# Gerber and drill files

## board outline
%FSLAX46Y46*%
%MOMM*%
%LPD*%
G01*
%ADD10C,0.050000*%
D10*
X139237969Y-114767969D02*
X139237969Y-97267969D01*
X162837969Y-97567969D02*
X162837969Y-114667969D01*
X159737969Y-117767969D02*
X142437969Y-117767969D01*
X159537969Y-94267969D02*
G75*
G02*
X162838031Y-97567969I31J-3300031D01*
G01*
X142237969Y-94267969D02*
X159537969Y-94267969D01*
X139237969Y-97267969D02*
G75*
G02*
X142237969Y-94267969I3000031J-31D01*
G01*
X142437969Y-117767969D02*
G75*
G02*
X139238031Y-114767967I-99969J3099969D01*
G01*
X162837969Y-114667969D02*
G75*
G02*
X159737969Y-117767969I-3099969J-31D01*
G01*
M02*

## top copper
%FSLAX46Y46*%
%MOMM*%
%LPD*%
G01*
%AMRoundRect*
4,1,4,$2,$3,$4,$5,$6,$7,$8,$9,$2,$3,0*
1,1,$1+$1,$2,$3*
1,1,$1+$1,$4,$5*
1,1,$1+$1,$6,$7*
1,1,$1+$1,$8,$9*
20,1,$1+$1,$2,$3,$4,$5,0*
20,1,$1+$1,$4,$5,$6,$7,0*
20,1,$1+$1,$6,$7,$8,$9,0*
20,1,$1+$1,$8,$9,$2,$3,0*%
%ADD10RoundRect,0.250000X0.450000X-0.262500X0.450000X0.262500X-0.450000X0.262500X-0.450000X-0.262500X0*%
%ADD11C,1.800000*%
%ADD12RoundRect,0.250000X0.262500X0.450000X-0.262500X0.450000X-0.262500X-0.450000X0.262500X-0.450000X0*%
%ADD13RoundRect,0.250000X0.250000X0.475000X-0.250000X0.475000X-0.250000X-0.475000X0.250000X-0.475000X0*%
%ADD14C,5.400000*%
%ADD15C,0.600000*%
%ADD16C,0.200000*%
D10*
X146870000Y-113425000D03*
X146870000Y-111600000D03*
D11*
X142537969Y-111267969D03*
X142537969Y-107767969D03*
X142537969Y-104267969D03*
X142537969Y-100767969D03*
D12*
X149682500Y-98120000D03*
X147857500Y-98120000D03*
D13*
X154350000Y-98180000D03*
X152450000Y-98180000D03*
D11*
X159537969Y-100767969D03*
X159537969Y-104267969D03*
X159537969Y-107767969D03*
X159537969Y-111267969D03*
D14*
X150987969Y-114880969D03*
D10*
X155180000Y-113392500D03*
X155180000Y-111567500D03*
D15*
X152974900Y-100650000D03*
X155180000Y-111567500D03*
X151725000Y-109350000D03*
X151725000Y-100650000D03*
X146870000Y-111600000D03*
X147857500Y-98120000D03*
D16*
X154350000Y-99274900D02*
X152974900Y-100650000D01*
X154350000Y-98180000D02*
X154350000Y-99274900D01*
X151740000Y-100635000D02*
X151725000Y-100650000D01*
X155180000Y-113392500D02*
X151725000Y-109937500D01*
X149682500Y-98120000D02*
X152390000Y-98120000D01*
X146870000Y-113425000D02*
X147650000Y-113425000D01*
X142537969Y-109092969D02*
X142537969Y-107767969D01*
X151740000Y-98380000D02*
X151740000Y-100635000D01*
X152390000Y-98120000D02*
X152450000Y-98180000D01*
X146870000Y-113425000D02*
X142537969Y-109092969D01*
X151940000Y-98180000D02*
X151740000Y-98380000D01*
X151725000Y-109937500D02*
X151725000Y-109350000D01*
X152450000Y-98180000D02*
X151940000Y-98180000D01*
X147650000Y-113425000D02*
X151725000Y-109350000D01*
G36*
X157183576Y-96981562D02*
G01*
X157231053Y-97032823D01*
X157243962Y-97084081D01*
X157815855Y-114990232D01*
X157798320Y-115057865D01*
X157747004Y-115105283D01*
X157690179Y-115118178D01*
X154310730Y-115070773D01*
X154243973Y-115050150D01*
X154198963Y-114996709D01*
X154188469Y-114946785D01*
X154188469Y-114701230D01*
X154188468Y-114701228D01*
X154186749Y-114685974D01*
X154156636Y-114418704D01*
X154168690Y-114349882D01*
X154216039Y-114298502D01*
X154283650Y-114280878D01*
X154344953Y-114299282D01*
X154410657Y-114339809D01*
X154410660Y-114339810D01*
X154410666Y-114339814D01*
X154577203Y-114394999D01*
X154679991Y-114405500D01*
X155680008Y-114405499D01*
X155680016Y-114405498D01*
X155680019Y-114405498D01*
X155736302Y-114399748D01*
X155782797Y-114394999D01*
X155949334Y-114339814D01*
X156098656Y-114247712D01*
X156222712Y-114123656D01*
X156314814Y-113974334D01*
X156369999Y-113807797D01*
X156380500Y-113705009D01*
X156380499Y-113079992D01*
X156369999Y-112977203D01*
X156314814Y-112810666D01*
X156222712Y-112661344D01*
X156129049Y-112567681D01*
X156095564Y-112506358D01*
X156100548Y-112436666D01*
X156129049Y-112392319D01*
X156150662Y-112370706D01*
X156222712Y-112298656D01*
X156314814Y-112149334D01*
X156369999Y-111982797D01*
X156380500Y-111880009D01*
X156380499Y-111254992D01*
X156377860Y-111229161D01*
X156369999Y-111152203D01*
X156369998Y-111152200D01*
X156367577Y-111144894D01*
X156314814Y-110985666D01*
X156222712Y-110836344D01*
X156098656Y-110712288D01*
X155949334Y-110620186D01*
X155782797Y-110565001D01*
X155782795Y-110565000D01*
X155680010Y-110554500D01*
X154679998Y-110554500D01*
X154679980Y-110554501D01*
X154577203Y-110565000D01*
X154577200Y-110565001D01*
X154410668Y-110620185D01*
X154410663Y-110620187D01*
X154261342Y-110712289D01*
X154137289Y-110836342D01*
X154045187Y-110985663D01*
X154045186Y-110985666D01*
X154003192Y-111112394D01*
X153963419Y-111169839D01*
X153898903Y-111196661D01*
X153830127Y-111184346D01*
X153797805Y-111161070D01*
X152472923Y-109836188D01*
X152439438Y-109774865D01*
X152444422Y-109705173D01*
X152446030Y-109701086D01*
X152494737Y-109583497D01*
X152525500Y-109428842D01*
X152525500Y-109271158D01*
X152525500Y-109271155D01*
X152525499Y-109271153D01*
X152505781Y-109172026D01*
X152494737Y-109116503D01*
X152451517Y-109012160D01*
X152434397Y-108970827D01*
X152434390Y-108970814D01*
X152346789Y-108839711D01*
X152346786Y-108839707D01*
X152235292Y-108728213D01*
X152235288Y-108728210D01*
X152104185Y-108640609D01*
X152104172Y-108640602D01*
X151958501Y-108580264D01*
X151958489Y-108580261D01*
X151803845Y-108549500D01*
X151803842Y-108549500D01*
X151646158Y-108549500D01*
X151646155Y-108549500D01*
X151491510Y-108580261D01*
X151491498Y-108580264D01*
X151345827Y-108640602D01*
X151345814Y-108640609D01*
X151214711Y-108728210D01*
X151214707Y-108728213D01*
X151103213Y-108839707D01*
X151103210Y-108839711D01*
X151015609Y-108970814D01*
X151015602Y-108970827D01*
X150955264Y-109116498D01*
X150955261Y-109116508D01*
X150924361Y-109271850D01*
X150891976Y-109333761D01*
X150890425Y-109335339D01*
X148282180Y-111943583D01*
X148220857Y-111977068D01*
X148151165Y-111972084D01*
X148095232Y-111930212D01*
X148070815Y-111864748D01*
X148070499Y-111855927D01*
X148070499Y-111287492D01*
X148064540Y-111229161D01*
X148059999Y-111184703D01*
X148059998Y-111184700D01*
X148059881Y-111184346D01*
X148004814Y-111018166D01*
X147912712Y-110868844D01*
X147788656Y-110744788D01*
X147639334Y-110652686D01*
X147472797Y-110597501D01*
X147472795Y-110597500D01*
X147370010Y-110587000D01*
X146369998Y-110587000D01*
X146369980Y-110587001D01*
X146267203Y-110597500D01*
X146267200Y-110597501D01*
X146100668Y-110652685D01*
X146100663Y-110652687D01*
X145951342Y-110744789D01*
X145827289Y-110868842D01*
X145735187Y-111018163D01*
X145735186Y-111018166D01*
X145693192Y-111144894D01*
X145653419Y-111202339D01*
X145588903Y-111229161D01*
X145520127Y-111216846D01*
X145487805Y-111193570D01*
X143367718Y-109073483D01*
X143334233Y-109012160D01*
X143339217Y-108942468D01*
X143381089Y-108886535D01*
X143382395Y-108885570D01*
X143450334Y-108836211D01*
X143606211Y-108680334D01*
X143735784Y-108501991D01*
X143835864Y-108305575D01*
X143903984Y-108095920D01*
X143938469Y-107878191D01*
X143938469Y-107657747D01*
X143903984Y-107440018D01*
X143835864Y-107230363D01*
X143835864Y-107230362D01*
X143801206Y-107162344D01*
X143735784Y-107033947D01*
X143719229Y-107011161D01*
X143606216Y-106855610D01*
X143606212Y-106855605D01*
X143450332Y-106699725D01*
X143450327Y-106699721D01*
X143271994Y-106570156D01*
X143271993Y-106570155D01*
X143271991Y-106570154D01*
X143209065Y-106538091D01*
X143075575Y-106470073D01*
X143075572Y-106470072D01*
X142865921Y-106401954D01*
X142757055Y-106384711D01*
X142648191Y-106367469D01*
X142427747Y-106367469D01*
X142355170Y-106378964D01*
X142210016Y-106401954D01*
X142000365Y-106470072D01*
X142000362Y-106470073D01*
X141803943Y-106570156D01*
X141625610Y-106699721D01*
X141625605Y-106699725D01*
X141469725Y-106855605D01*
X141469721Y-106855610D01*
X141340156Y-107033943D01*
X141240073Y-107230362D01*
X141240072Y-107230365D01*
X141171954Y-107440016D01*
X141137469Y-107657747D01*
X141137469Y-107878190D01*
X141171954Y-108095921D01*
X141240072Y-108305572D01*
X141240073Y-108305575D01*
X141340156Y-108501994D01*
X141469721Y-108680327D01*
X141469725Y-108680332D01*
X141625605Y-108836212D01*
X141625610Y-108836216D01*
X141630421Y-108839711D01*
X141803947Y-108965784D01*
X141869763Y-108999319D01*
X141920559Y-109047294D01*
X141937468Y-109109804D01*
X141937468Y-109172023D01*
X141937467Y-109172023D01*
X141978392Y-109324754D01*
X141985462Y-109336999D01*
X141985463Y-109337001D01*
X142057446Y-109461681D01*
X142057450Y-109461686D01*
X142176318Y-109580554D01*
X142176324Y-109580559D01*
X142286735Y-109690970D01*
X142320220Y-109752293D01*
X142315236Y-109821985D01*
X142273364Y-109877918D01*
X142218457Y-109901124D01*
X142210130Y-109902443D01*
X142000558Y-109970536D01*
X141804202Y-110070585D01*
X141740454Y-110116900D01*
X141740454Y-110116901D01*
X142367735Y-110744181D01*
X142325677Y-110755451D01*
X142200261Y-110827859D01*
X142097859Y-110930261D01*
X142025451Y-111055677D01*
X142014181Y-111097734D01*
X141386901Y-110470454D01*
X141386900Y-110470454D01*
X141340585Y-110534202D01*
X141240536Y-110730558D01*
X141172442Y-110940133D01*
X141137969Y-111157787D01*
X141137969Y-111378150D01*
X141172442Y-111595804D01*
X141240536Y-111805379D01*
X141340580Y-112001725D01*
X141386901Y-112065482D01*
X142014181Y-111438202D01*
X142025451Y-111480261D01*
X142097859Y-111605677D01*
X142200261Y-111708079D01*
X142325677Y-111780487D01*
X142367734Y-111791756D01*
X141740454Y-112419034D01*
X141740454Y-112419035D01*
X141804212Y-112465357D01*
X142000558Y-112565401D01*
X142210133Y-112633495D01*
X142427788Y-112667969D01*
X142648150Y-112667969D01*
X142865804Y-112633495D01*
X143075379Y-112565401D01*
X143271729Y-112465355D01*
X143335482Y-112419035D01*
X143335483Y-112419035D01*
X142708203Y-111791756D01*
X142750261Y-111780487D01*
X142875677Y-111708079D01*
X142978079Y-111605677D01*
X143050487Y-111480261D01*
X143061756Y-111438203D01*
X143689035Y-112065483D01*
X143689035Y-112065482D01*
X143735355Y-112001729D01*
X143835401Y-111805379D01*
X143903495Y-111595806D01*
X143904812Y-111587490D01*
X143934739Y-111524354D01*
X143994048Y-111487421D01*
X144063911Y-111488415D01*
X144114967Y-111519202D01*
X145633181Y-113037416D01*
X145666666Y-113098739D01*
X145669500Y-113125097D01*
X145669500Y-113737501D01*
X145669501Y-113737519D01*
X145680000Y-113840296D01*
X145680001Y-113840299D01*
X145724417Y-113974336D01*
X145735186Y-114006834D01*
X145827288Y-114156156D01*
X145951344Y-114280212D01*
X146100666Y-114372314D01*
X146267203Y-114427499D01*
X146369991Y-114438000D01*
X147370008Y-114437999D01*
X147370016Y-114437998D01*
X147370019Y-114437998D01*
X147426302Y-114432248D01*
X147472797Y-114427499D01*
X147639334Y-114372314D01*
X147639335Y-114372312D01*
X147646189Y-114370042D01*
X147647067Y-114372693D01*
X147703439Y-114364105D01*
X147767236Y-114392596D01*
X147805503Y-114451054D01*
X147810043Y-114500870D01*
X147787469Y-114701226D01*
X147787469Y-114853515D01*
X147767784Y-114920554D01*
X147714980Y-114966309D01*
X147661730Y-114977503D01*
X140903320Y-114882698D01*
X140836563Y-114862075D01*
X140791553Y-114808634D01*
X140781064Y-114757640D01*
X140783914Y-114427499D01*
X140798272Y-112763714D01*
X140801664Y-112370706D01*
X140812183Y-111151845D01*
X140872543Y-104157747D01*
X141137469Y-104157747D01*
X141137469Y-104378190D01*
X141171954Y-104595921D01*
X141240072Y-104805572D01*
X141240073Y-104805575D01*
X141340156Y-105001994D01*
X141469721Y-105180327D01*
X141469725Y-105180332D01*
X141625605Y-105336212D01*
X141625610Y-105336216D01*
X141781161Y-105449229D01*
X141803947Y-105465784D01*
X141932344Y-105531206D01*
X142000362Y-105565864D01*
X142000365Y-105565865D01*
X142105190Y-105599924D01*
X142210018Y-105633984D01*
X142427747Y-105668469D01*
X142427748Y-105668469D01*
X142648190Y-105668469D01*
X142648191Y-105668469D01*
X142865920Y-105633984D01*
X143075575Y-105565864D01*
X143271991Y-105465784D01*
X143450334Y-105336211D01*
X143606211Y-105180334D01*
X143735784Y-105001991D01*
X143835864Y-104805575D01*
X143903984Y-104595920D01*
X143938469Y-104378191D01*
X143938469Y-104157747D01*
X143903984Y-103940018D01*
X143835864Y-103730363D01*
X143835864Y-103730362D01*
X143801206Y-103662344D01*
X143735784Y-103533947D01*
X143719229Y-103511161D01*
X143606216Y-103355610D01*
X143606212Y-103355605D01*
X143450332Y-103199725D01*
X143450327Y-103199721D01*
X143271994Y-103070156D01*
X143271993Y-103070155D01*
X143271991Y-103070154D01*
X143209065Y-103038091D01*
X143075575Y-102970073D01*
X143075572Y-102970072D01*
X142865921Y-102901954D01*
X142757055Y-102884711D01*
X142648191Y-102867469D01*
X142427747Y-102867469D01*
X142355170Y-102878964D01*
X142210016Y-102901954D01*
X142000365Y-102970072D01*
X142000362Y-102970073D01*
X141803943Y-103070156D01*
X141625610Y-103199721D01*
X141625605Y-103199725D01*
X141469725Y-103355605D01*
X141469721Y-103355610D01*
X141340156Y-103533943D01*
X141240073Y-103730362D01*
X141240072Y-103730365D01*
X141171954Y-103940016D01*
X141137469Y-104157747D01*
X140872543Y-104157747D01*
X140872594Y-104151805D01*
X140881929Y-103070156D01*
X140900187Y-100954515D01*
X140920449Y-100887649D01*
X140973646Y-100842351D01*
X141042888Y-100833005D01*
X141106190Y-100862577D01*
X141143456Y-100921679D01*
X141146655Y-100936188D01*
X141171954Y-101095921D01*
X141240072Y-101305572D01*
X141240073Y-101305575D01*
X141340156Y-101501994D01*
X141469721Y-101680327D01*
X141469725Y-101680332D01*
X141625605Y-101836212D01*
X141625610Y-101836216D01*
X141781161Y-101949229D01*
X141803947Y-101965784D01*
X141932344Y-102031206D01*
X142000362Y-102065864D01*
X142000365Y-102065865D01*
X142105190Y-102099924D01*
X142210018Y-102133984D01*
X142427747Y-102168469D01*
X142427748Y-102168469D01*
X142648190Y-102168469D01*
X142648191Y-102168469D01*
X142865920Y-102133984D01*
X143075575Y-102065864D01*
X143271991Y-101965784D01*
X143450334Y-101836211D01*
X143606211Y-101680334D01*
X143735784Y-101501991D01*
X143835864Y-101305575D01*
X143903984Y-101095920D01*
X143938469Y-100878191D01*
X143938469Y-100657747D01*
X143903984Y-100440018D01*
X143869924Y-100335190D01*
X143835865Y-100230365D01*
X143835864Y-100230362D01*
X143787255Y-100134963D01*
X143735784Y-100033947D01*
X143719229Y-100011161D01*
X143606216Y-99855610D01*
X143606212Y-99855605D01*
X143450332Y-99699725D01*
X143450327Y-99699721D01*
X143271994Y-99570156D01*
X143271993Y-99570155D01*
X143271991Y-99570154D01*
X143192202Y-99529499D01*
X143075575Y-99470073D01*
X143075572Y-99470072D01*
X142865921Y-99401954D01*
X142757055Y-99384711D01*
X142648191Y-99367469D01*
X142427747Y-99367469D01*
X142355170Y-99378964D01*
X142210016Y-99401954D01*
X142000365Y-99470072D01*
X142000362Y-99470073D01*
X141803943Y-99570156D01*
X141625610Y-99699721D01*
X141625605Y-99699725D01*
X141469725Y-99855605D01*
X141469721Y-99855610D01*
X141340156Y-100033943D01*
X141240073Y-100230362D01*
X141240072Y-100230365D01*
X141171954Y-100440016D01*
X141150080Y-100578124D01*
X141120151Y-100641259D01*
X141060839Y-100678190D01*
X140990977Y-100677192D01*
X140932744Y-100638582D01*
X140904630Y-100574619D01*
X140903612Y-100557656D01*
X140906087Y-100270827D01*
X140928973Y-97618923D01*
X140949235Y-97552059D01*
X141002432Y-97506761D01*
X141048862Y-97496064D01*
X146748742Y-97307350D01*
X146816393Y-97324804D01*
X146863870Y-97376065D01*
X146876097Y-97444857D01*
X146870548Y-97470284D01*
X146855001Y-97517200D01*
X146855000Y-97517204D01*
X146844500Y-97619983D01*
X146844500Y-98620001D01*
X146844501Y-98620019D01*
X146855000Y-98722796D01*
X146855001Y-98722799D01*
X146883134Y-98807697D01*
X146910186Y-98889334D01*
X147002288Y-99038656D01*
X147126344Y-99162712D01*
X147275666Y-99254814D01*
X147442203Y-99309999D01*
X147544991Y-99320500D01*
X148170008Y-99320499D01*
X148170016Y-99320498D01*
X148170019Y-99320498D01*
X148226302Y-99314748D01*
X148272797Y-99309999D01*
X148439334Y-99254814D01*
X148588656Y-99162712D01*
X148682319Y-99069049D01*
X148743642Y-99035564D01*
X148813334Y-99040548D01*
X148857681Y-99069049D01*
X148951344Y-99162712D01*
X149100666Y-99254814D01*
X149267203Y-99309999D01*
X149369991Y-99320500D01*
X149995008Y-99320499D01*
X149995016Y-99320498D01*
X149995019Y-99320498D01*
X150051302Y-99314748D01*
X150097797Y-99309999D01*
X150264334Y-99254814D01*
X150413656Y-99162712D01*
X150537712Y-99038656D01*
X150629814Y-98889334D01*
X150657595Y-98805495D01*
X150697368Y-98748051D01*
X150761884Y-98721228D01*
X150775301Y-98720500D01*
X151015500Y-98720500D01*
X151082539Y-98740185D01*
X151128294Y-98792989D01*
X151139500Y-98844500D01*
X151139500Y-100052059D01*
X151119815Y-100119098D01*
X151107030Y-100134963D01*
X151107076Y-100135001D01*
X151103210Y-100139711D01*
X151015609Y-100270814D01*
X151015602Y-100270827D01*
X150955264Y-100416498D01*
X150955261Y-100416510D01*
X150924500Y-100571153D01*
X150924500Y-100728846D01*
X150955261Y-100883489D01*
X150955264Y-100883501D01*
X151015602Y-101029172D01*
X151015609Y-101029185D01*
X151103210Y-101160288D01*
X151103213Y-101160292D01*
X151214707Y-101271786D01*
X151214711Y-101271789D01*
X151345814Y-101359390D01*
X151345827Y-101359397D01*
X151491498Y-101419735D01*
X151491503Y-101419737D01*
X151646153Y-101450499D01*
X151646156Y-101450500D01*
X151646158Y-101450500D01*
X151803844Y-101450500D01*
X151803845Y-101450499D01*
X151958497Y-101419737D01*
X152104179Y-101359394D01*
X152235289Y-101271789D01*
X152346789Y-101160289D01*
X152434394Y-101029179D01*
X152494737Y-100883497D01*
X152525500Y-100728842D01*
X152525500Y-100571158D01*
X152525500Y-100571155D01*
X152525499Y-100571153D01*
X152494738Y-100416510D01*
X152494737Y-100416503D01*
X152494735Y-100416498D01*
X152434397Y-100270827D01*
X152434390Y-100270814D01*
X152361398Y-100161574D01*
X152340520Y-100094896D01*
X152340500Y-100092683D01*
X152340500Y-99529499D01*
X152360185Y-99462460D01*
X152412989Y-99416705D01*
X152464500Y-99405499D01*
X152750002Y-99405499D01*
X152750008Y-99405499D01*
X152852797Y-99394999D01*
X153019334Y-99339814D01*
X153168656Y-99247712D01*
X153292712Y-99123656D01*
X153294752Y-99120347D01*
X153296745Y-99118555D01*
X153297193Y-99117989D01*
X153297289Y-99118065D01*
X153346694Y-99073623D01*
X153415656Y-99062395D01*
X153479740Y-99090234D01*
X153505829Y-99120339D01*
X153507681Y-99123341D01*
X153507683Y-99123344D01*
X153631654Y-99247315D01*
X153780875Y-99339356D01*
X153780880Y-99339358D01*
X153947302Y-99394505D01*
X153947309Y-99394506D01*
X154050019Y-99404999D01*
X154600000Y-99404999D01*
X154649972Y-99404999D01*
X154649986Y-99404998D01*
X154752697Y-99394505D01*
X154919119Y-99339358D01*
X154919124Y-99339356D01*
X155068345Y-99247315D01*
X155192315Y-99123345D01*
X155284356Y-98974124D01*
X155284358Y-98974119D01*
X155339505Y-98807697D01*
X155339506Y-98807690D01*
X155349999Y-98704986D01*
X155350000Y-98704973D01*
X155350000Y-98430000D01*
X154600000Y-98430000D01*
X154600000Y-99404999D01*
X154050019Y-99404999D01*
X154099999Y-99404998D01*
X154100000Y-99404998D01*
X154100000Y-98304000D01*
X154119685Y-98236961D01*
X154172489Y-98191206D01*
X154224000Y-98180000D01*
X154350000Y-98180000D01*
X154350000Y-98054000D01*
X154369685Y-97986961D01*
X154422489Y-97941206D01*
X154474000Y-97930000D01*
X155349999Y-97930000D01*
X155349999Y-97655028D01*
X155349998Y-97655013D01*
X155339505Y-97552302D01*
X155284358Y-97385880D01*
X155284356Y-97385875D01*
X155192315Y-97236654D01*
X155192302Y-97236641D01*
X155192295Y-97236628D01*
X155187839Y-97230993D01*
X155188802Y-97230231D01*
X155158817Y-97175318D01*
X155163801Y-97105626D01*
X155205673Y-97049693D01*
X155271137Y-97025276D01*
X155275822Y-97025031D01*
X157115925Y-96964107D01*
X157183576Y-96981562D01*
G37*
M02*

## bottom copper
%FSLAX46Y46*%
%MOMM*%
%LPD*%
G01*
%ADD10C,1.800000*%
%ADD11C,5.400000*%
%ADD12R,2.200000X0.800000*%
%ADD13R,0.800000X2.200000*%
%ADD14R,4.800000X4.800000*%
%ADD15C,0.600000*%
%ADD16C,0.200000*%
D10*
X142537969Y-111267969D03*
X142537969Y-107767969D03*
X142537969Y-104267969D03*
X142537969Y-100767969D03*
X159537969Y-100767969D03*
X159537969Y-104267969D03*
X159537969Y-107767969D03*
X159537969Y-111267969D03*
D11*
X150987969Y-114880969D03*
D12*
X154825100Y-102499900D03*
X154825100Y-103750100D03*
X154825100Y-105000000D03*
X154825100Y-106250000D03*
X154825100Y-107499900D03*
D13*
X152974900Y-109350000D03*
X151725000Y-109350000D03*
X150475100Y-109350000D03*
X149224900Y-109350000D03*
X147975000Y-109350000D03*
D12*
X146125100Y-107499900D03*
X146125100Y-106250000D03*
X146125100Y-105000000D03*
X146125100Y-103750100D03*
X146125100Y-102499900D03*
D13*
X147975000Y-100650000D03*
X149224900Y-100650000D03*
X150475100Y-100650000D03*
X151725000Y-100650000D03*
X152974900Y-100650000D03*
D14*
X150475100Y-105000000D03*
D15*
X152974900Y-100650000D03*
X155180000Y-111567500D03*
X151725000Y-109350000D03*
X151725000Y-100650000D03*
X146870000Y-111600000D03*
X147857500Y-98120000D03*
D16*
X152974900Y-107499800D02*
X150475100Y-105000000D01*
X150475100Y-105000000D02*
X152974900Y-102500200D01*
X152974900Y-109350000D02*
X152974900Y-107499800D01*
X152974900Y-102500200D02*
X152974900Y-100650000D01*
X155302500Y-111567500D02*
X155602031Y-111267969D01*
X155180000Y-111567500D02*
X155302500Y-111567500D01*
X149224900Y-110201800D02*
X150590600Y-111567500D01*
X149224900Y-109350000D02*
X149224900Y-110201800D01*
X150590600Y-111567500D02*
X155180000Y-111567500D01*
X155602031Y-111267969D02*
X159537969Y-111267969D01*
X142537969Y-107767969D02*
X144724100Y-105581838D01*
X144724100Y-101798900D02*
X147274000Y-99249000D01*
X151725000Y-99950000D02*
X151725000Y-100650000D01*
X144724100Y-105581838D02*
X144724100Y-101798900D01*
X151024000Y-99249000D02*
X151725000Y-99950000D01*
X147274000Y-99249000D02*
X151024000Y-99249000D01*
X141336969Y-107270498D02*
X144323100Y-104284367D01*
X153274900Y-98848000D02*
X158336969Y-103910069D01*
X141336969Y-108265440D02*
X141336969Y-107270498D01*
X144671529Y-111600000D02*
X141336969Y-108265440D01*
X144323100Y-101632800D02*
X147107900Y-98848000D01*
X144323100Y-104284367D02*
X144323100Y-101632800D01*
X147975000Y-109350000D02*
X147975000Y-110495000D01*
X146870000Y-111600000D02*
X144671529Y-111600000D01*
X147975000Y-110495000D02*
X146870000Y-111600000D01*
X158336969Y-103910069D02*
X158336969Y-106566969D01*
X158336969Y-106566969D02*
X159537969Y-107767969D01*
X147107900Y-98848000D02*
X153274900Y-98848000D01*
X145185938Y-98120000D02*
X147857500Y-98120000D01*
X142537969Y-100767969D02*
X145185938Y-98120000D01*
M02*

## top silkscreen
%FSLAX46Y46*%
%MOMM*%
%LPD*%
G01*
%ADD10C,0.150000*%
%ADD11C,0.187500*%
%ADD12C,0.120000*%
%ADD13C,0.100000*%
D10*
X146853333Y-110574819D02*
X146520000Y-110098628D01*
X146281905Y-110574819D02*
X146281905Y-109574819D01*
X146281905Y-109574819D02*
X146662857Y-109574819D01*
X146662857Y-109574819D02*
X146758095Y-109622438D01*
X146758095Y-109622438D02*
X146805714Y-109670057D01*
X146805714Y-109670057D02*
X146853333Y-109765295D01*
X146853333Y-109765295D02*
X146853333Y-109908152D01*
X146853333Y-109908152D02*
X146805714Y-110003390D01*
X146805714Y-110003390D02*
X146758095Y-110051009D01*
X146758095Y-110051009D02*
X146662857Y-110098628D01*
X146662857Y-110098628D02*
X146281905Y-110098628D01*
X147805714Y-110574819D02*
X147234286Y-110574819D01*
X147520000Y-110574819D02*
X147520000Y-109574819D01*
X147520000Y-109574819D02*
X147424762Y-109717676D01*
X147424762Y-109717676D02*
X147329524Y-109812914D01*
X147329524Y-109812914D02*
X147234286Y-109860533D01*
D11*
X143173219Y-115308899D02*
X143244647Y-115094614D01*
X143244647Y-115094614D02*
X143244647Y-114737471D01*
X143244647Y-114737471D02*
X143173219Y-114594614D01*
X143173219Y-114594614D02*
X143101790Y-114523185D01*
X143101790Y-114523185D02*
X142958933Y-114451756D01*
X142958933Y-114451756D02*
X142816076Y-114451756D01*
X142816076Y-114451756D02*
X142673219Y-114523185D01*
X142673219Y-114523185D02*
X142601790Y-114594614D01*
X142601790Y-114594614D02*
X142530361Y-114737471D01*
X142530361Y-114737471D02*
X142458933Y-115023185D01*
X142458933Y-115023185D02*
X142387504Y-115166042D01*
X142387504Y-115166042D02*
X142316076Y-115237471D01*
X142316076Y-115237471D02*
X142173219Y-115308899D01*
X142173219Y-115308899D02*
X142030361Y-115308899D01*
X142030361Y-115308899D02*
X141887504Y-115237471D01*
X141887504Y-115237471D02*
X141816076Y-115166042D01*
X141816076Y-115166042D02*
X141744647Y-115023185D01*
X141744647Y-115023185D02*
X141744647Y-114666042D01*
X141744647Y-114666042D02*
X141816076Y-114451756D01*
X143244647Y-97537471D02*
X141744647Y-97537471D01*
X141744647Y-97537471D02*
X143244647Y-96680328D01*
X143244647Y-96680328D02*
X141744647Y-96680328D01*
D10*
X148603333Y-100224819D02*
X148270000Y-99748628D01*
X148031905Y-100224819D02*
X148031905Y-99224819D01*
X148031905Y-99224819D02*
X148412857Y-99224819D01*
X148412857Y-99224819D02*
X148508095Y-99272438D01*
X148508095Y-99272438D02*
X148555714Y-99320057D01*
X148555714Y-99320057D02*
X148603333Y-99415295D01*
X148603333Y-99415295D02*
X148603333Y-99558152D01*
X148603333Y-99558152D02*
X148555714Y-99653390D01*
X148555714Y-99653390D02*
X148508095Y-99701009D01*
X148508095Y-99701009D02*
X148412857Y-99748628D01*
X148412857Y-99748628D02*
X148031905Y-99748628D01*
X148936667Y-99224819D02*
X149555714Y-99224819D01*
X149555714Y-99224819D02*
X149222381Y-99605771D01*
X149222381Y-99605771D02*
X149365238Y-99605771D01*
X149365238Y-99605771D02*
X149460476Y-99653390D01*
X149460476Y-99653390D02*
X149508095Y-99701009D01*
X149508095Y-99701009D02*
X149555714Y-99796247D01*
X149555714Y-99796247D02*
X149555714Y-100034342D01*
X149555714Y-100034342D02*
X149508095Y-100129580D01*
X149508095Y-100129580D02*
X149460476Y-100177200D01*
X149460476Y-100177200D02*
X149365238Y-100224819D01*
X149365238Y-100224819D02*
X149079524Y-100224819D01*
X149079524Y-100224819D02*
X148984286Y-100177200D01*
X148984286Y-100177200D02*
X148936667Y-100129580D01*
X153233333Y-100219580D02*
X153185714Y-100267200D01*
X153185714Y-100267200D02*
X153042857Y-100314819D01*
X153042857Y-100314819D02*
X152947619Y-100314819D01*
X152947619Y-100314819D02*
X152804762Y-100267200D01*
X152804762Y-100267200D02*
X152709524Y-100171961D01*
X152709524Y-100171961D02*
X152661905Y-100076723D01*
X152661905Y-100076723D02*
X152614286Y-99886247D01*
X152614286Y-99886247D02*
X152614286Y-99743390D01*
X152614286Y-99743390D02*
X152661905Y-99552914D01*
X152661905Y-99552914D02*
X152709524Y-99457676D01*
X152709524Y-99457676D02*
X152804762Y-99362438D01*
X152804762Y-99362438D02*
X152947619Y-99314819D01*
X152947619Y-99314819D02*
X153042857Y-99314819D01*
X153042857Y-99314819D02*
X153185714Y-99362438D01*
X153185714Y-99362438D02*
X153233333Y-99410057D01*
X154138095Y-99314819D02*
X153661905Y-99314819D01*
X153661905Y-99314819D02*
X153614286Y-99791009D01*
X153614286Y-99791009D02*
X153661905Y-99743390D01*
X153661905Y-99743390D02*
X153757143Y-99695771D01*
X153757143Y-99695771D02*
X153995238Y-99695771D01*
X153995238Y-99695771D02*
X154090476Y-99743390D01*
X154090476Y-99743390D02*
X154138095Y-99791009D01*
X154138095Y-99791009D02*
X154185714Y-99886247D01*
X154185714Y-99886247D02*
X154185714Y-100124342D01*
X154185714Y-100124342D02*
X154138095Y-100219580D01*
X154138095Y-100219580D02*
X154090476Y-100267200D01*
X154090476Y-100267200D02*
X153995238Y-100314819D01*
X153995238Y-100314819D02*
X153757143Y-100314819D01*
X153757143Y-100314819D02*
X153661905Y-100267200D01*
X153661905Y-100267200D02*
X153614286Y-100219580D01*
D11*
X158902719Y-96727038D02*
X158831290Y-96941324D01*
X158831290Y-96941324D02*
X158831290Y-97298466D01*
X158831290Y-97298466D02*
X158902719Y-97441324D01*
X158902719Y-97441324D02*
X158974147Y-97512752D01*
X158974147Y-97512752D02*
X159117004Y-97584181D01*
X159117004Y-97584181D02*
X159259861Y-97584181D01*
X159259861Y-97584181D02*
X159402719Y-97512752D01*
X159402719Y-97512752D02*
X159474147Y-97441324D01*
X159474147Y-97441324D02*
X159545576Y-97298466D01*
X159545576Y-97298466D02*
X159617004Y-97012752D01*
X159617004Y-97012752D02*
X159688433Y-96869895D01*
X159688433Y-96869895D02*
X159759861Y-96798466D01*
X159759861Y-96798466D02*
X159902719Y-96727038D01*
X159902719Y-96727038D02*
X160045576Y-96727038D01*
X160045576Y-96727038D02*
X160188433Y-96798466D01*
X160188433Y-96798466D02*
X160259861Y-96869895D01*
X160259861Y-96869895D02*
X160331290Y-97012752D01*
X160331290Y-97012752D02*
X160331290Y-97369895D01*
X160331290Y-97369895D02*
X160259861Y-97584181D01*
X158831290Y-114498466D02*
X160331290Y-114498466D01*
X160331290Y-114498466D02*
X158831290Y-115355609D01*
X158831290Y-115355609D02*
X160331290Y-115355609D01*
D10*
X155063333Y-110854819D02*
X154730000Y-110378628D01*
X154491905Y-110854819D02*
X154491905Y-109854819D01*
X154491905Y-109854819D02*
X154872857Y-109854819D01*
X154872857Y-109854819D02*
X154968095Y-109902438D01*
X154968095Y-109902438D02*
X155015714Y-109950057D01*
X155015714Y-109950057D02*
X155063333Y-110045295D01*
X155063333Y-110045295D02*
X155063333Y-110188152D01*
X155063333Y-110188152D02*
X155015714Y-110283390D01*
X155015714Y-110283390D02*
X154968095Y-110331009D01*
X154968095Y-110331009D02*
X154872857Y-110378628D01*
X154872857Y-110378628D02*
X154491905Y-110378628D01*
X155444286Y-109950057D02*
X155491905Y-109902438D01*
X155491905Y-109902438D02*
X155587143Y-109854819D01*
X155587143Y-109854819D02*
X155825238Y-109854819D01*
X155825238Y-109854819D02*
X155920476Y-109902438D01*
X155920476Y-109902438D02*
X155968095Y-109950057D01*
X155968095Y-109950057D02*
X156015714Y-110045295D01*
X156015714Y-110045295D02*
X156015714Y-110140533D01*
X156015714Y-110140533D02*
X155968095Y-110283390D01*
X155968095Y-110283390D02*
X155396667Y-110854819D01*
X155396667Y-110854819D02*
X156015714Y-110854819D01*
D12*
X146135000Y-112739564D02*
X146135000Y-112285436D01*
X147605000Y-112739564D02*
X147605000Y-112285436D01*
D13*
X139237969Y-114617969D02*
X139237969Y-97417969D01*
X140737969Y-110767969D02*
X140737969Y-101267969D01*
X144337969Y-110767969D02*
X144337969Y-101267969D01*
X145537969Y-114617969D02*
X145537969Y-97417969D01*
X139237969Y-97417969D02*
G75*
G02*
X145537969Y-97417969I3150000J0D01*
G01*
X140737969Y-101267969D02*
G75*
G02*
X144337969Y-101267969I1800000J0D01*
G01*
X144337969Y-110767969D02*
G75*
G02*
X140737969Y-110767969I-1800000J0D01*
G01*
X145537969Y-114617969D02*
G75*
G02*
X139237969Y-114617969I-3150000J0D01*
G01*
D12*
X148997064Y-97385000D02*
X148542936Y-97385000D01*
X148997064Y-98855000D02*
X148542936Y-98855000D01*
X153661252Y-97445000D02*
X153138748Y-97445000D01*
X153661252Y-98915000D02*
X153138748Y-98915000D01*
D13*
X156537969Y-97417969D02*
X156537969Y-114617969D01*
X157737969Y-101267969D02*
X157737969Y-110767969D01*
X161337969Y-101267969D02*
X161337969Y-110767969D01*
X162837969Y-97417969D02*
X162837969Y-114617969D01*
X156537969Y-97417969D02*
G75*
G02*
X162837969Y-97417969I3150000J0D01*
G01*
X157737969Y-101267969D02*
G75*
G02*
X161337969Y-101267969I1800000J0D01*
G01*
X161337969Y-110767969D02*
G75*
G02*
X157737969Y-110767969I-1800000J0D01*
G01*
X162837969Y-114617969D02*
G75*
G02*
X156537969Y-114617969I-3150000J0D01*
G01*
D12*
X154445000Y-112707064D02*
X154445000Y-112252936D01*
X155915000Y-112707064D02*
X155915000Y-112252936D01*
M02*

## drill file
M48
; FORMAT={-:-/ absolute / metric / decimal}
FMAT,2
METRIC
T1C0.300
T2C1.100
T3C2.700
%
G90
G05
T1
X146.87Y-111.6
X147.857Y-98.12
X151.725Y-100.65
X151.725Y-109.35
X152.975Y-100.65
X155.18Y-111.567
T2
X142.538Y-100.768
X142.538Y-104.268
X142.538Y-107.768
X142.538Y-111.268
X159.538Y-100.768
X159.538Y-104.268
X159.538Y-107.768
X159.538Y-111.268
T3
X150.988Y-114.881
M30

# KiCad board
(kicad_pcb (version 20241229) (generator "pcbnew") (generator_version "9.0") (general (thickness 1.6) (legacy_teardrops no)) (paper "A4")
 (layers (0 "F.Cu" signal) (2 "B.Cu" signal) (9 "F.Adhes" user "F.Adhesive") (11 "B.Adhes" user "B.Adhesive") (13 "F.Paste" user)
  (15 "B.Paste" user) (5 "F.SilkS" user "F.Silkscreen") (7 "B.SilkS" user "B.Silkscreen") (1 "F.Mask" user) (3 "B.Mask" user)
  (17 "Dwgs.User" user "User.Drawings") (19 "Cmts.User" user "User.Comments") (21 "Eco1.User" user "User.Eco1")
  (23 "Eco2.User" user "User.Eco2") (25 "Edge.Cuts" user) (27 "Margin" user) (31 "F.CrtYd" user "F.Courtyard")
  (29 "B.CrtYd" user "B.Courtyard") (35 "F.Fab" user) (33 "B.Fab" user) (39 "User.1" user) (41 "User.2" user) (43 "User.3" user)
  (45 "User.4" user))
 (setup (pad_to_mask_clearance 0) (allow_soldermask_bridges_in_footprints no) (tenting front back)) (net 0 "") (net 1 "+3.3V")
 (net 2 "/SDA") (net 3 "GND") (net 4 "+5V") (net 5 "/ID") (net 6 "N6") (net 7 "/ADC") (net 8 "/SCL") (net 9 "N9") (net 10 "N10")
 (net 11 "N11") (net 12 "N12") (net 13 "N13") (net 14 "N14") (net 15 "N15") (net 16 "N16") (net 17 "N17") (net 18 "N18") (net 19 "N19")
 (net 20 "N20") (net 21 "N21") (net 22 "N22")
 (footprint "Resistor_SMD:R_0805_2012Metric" (layer "F.Cu") (at 146.87 112.5125 90)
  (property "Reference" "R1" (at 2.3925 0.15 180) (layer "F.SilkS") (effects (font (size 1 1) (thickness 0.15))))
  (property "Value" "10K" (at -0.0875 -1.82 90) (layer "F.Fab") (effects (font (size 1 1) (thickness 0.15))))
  (fp_line (start -0.227064 -0.735) (end 0.227064 -0.735) (stroke (width 0.12) (type solid)) (layer "F.SilkS"))
  (fp_line (start -0.227064 0.735) (end 0.227064 0.735) (stroke (width 0.12) (type solid)) (layer "F.SilkS"))
  (pad "1" smd roundrect (at -0.9125 0 90) (size 1.025 1.4) (layers "F.Cu" "F.Mask" "F.Paste") (roundrect_rratio 0.243902) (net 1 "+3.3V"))
  (pad "2" smd roundrect (at 0.9125 0 90) (size 1.025 1.4) (layers "F.Cu" "F.Mask" "F.Paste") (roundrect_rratio 0.243902) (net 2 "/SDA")))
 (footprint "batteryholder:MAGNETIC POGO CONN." (layer "F.Cu") (at 142.537969 106.017969 90)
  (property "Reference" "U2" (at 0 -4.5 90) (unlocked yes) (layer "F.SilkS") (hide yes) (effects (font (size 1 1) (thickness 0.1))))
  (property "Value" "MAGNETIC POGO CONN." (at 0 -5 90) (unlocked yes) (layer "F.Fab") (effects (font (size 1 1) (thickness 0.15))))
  (fp_line (start -8.6 -3.3) (end 8.6 -3.3) (stroke (width 0.1) (type default)) (layer "F.SilkS"))
  (fp_line (start -4.75 -1.8) (end 4.75 -1.8) (stroke (width 0.1) (type default)) (layer "F.SilkS"))
  (fp_line (start -4.75 1.8) (end 4.75 1.8) (stroke (width 0.1) (type default)) (layer "F.SilkS"))
  (fp_line (start -8.6 3) (end 8.6 3) (stroke (width 0.1) (type default)) (layer "F.SilkS"))
  (fp_arc (start 8.6 -3.3) (mid 11.75 -0.15) (end 8.6 3) (stroke (width 0.1) (type default)) (layer "F.SilkS"))
  (fp_arc (start 4.75 -1.8) (mid 6.55 0) (end 4.75 1.8) (stroke (width 0.1) (type default)) (layer "F.SilkS"))
  (fp_arc (start -4.75 1.8) (mid -6.55 0) (end -4.75 -1.8) (stroke (width 0.1) (type default)) (layer "F.SilkS"))
  (fp_arc (start -8.6 3) (mid -11.75 -0.15) (end -8.6 -3.3) (stroke (width 0.1) (type default)) (layer "F.SilkS"))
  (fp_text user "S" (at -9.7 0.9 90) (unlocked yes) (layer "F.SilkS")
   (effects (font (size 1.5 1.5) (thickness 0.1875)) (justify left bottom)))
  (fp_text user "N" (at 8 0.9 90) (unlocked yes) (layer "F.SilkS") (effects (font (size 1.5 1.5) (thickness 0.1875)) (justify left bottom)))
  (pad "1" thru_hole circle (at -5.25 0 90) (size 1.8 1.8) (drill 1.1) (layers "*.Cu" "*.Mask") (remove_unused_layers no) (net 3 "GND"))
  (pad "2" thru_hole circle (at -1.75 0 90) (size 1.8 1.8) (drill 1.1) (layers "*.Cu" "*.Mask") (remove_unused_layers no) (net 1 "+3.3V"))
  (pad "3" thru_hole circle (at 1.75 0 90) (size 1.8 1.8) (drill 1.1) (layers "*.Cu" "*.Mask") (remove_unused_layers no) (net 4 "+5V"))
  (pad "4" thru_hole circle (at 5.25 0 90) (size 1.8 1.8) (drill 1.1) (layers "*.Cu" "*.Mask") (remove_unused_layers no) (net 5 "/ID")))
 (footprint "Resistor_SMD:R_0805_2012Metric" (layer "F.Cu") (at 148.77 98.12 180)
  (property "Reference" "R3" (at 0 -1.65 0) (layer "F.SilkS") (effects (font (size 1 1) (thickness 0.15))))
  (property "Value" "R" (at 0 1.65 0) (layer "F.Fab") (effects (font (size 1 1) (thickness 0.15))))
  (fp_line (start -0.227064 0.735) (end 0.227064 0.735) (stroke (width 0.12) (type solid)) (layer "F.SilkS"))
  (fp_line (start -0.227064 -0.735) (end 0.227064 -0.735) (stroke (width 0.12) (type solid)) (layer "F.SilkS"))
  (pad "1" smd roundrect (at -0.9125 0 180) (size 1.025 1.4) (layers "F.Cu" "F.Mask" "F.Paste") (roundrect_rratio 0.243902) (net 1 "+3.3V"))
  (pad "2" smd roundrect (at 0.9125 0 180) (size 1.025 1.4) (layers "F.Cu" "F.Mask" "F.Paste") (roundrect_rratio 0.243902) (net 5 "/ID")))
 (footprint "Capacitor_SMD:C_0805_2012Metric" (layer "F.Cu") (at 153.4 98.18 180)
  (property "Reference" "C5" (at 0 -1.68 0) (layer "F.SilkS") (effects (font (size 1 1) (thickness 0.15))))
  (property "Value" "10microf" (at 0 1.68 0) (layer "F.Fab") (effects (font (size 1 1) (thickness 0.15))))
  (fp_line (start -0.261252 0.735) (end 0.261252 0.735) (stroke (width 0.12) (type solid)) (layer "F.SilkS"))
  (fp_line (start -0.261252 -0.735) (end 0.261252 -0.735) (stroke (width 0.12) (type solid)) (layer "F.SilkS"))
  (pad "1" smd roundrect (at -0.95 0 180) (size 1 1.45) (layers "F.Cu" "F.Mask" "F.Paste") (roundrect_rratio 0.25) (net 3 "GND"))
  (pad "2" smd roundrect (at 0.95 0 180) (size 1 1.45) (layers "F.Cu" "F.Mask" "F.Paste") (roundrect_rratio 0.25) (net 1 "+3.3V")))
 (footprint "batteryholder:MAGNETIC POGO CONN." (layer "F.Cu") (at 159.537969 106.017969 -90)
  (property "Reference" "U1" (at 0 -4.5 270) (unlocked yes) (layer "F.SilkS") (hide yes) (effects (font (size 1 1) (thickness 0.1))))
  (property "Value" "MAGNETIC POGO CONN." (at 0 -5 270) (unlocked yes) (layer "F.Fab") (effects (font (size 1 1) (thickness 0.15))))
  (fp_line (start -8.6 3) (end 8.6 3) (stroke (width 0.1) (type default)) (layer "F.SilkS"))
  (fp_line (start -4.75 1.8) (end 4.75 1.8) (stroke (width 0.1) (type default)) (layer "F.SilkS"))
  (fp_line (start -4.75 -1.8) (end 4.75 -1.8) (stroke (width 0.1) (type default)) (layer "F.SilkS"))
  (fp_line (start -8.6 -3.3) (end 8.6 -3.3) (stroke (width 0.1) (type default)) (layer "F.SilkS"))
  (fp_arc (start -8.6 3) (mid -11.75 -0.15) (end -8.6 -3.3) (stroke (width 0.1) (type default)) (layer "F.SilkS"))
  (fp_arc (start -4.75 1.8) (mid -6.55 0) (end -4.75 -1.8) (stroke (width 0.1) (type default)) (layer "F.SilkS"))
  (fp_arc (start 4.75 -1.8) (mid 6.55 0) (end 4.75 1.8) (stroke (width 0.1) (type default)) (layer "F.SilkS"))
  (fp_arc (start 8.6 -3.3) (mid 11.75 -0.15) (end 8.6 3) (stroke (width 0.1) (type default)) (layer "F.SilkS"))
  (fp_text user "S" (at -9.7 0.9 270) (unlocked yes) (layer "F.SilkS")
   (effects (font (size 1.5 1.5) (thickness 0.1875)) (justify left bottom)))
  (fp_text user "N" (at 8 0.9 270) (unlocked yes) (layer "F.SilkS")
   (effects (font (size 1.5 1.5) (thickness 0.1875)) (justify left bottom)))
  (pad "1" thru_hole circle (at -5.25 0 270) (size 1.8 1.8) (drill 1.1) (layers "*.Cu" "*.Mask") (remove_unused_layers no) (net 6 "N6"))
  (pad "2" thru_hole circle (at -1.75 0 270) (size 1.8 1.8) (drill 1.1) (layers "*.Cu" "*.Mask") (remove_unused_layers no) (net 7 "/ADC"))
  (pad "3" thru_hole circle (at 1.75 0 270) (size 1.8 1.8) (drill 1.1) (layers "*.Cu" "*.Mask") (remove_unused_layers no) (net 2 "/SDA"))
  (pad "4" thru_hole circle (at 5.25 0 270) (size 1.8 1.8) (drill 1.1) (layers "*.Cu" "*.Mask") (remove_unused_layers no) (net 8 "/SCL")))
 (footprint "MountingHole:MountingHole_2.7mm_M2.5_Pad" (layer "F.Cu") (at 150.987969 114.880969)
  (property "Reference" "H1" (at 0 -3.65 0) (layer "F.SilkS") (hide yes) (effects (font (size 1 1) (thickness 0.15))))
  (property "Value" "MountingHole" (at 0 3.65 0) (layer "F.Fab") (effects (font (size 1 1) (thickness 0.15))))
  (pad "1" thru_hole circle (at 0 0) (size 5.4 5.4) (drill 2.7) (layers "*.Cu" "*.Mask") (remove_unused_layers no) (zone_connect 2)))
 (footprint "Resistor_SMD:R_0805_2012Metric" (layer "F.Cu") (at 155.18 112.48 90)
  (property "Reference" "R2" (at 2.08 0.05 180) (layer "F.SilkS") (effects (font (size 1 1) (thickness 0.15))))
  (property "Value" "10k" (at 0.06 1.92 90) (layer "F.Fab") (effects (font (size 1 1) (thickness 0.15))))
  (fp_line (start -0.227064 -0.735) (end 0.227064 -0.735) (stroke (width 0.12) (type solid)) (layer "F.SilkS"))
  (fp_line (start -0.227064 0.735) (end 0.227064 0.735) (stroke (width 0.12) (type solid)) (layer "F.SilkS"))
  (pad "1" smd roundrect (at -0.9125 0 90) (size 1.025 1.4) (layers "F.Cu" "F.Mask" "F.Paste") (roundrect_rratio 0.243902) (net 1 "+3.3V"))
  (pad "2" smd roundrect (at 0.9125 0 90) (size 1.025 1.4) (layers "F.Cu" "F.Mask" "F.Paste") (roundrect_rratio 0.243902) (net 8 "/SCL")))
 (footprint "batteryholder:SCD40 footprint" (layer "B.Cu") (at 150.475 105 180)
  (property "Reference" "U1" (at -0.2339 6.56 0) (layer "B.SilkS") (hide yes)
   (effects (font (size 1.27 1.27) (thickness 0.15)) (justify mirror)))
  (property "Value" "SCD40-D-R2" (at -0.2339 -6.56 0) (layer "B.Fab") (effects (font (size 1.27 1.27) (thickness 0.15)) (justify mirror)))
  (pad "1" smd rect (at -4.3501 2.5001 180) (size 2.2 0.8) (layers "B.Cu" "B.Mask" "B.Paste") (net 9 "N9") (solder_mask_margin 0.05)
   (solder_paste_margin 0) (thermal_bridge_angle 0))
  (pad "2" smd rect (at -4.3501 1.2499 180) (size 2.2 0.8) (layers "B.Cu" "B.Mask" "B.Paste") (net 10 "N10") (solder_mask_margin 0.05)
   (solder_paste_margin 0) (thermal_bridge_angle 0))
  (pad "3" smd rect (at -4.3501 0 180) (size 2.2 0.8) (layers "B.Cu" "B.Mask" "B.Paste") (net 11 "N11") (solder_mask_margin 0.05)
   (solder_paste_margin 0) (thermal_bridge_angle 0))
  (pad "4" smd rect (at -4.3501 -1.25 180) (size 2.2 0.8) (layers "B.Cu" "B.Mask" "B.Paste") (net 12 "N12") (solder_mask_margin 0.05)
   (solder_paste_margin 0) (thermal_bridge_angle 0))
  (pad "5" smd rect (at -4.3501 -2.4999 180) (size 2.2 0.8) (layers "B.Cu" "B.Mask" "B.Paste") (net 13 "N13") (solder_mask_margin 0.05)
   (solder_paste_margin 0) (thermal_bridge_angle 0))
  (pad "6" smd rect (at -2.4999 -4.35 90) (size 2.2 0.8) (layers "B.Cu" "B.Mask" "B.Paste") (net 3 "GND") (solder_mask_margin 0.05)
   (solder_paste_margin 0) (thermal_bridge_angle 0))
  (pad "7" smd rect (at -1.25 -4.35 90) (size 2.2 0.8) (layers "B.Cu" "B.Mask" "B.Paste") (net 1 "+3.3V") (solder_mask_margin 0.05)
   (solder_paste_margin 0) (thermal_bridge_angle 0))
  (pad "8" smd rect (at -0.0001 -4.35 90) (size 2.2 0.8) (layers "B.Cu" "B.Mask" "B.Paste") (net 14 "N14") (solder_mask_margin 0.05)
   (solder_paste_margin 0) (thermal_bridge_angle 0))
  (pad "9" smd rect (at 1.2501 -4.35 90) (size 2.2 0.8) (layers "B.Cu" "B.Mask" "B.Paste") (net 8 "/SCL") (solder_mask_margin 0.05)
   (solder_paste_margin 0) (thermal_bridge_angle 0))
  (pad "10" smd rect (at 2.5 -4.35 90) (size 2.2 0.8) (layers "B.Cu" "B.Mask" "B.Paste") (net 2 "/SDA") (solder_mask_margin 0.05)
   (solder_paste_margin 0) (thermal_bridge_angle 0))
  (pad "11" smd rect (at 4.3499 -2.4999) (size 2.2 0.8) (layers "B.Cu" "B.Mask" "B.Paste") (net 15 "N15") (solder_mask_margin 0.05)
   (solder_paste_margin 0) (thermal_bridge_angle 0))
  (pad "12" smd rect (at 4.3499 -1.25) (size 2.2 0.8) (layers "B.Cu" "B.Mask" "B.Paste") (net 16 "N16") (solder_mask_margin 0.05)
   (solder_paste_margin 0) (thermal_bridge_angle 0))
  (pad "13" smd rect (at 4.3499 0) (size 2.2 0.8) (layers "B.Cu" "B.Mask" "B.Paste") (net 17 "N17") (solder_mask_margin 0.05)
   (solder_paste_margin 0) (thermal_bridge_angle 0))
  (pad "14" smd rect (at 4.3499 1.2499) (size 2.2 0.8) (layers "B.Cu" "B.Mask" "B.Paste") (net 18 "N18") (solder_mask_margin 0.05)
   (solder_paste_margin 0) (thermal_bridge_angle 0))
  (pad "15" smd rect (at 4.3499 2.5001) (size 2.2 0.8) (layers "B.Cu" "B.Mask" "B.Paste") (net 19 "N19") (solder_mask_margin 0.05)
   (solder_paste_margin 0) (thermal_bridge_angle 0))
  (pad "16" smd rect (at 2.5 4.35 270) (size 2.2 0.8) (layers "B.Cu" "B.Mask" "B.Paste") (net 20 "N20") (solder_mask_margin 0.05)
   (solder_paste_margin 0) (thermal_bridge_angle 0))
  (pad "17" smd rect (at 1.2501 4.35 270) (size 2.2 0.8) (layers "B.Cu" "B.Mask" "B.Paste") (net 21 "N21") (solder_mask_margin 0.05)
   (solder_paste_margin 0) (thermal_bridge_angle 0))
  (pad "18" smd rect (at -0.0001 4.35 270) (size 2.2 0.8) (layers "B.Cu" "B.Mask" "B.Paste") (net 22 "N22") (solder_mask_margin 0.05)
   (solder_paste_margin 0) (thermal_bridge_angle 0))
  (pad "19" smd rect (at -1.25 4.35 270) (size 2.2 0.8) (layers "B.Cu" "B.Mask" "B.Paste") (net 1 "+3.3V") (solder_mask_margin 0.05)
   (solder_paste_margin 0) (thermal_bridge_angle 0))
  (pad "20" smd rect (at -2.4999 4.35 270) (size 2.2 0.8) (layers "B.Cu" "B.Mask" "B.Paste") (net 3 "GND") (solder_mask_margin 0.05)
   (solder_paste_margin 0) (thermal_bridge_angle 0))
  (pad "21" smd rect (at -0.0001 0 90) (size 4.8 4.8) (layers "B.Cu" "B.Mask" "B.Paste") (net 3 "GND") (solder_mask_margin 0.05)
   (solder_paste_margin 0) (thermal_bridge_angle 0))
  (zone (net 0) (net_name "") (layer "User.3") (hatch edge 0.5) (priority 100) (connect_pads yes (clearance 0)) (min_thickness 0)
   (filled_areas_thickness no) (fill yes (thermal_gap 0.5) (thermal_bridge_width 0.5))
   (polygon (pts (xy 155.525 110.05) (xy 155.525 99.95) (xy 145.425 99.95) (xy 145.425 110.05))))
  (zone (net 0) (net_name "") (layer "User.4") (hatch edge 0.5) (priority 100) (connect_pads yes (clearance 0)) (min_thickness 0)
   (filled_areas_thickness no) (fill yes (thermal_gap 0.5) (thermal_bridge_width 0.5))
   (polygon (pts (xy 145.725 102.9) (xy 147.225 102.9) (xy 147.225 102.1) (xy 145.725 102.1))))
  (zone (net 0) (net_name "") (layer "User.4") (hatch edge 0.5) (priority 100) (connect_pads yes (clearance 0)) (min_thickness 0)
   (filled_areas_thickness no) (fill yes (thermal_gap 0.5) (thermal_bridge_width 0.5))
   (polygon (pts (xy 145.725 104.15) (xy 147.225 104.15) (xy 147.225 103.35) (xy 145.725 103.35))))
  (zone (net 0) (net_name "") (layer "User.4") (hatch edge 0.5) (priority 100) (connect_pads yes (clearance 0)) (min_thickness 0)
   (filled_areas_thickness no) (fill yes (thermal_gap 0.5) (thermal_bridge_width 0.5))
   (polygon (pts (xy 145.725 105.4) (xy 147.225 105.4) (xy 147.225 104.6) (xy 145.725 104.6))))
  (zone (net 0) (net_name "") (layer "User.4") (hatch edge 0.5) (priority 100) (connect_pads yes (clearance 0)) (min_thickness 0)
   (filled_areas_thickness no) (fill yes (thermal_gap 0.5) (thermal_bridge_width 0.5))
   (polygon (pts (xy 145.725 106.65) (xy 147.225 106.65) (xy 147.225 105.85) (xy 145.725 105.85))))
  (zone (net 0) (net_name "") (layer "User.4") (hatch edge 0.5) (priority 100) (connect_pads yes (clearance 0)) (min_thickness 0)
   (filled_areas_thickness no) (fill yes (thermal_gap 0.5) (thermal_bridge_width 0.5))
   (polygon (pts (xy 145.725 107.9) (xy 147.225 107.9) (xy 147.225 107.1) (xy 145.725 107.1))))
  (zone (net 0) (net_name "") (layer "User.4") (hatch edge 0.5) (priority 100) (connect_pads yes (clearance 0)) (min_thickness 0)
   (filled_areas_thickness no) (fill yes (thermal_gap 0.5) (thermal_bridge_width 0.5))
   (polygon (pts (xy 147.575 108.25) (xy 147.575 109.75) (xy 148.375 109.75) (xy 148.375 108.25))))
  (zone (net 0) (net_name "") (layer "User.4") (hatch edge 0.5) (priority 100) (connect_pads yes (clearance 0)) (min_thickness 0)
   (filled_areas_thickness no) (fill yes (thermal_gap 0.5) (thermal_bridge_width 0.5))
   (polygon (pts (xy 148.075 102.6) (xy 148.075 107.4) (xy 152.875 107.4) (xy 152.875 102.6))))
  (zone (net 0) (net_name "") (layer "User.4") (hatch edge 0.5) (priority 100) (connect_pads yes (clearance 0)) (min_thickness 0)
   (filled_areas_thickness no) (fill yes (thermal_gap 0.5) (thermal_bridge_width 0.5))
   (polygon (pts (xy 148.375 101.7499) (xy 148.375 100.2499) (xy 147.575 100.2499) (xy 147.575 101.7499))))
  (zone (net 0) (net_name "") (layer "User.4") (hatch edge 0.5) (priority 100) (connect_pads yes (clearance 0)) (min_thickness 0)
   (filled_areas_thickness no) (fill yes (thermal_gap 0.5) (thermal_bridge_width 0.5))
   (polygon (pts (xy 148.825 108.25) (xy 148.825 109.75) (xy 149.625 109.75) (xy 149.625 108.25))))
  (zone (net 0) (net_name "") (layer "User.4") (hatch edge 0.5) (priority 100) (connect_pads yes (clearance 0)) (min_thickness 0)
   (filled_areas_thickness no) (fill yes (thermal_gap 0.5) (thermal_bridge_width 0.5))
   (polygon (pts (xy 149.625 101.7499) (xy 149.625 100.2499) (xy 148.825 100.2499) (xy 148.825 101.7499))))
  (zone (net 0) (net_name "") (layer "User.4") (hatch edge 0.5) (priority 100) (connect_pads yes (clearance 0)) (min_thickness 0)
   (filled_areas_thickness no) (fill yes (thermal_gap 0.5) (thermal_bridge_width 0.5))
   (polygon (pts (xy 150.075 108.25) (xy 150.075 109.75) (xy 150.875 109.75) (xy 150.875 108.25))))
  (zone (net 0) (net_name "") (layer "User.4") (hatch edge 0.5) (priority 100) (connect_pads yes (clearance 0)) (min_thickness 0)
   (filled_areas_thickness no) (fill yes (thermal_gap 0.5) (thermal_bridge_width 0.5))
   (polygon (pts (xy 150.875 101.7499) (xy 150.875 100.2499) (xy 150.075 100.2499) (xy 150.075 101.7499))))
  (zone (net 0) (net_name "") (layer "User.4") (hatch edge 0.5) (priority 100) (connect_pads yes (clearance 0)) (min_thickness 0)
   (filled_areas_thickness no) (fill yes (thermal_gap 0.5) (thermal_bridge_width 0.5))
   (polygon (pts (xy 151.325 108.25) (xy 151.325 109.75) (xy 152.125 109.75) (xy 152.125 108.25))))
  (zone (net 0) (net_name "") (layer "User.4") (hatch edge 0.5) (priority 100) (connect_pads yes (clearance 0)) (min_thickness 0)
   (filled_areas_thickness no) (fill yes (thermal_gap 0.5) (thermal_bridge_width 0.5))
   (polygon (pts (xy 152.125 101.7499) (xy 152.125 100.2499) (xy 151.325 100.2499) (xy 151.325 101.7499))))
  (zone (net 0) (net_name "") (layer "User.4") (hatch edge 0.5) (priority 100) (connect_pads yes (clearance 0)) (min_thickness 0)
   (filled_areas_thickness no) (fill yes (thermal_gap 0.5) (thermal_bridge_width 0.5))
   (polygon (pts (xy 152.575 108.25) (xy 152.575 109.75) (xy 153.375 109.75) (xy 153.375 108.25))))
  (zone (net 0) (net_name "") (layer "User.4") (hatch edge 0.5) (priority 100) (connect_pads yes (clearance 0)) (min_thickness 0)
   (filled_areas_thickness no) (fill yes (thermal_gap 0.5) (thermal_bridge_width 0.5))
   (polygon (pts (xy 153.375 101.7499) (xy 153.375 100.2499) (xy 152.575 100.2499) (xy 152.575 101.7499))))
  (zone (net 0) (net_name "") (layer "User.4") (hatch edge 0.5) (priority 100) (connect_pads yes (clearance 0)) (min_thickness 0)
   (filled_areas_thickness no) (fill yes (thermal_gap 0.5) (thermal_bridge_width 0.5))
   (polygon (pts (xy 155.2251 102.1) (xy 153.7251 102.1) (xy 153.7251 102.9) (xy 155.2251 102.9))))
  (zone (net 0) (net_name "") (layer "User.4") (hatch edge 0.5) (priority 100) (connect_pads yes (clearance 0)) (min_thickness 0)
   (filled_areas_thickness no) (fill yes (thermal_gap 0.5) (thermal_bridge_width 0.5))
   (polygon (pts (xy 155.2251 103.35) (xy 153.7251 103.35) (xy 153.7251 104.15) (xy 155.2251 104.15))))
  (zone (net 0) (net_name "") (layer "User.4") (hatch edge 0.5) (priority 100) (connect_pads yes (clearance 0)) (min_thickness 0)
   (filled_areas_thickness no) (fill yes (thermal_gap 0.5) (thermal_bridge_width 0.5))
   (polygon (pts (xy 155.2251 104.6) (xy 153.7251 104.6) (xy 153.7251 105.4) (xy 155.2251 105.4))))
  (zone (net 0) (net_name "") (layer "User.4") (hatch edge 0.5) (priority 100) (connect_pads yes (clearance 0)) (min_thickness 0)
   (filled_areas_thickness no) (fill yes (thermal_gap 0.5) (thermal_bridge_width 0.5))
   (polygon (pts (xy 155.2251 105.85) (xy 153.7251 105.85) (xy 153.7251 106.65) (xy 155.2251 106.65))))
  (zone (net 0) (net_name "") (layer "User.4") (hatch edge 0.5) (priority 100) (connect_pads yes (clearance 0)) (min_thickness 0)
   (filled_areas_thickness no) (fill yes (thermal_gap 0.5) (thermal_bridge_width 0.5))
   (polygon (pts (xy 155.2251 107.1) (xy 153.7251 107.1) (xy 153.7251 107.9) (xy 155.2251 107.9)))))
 (gr_line (start 139.237969 114.767969) (end 139.237969 97.267969) (stroke (width 0.05) (type default)) (layer "Edge.Cuts"))
 (gr_line (start 162.837969 97.567969) (end 162.837969 114.667969) (stroke (width 0.05) (type default)) (layer "Edge.Cuts"))
 (gr_line (start 159.737969 117.767969) (end 142.437969 117.767969) (stroke (width 0.05) (type solid)) (layer "Edge.Cuts"))
 (gr_arc (start 159.537969 94.267969) (mid 161.871421 95.234517) (end 162.837969 97.567969) (stroke (width 0.05) (type default))
  (layer "Edge.Cuts"))
 (gr_line (start 142.237969 94.267969) (end 159.537969 94.267969) (stroke (width 0.05) (type default)) (layer "Edge.Cuts"))
 (gr_arc (start 139.237969 97.267969) (mid 140.116649 95.146649) (end 142.237969 94.267969) (stroke (width 0.05) (type default))
  (layer "Edge.Cuts"))
 (gr_arc (start 142.437969 117.767969) (mid 140.216649 116.930711) (end 139.237969 114.767969) (stroke (width 0.05) (type default))
  (layer "Edge.Cuts"))
 (gr_arc (start 162.837969 114.667969) (mid 161.93 116.86) (end 159.737969 117.767969) (stroke (width 0.05) (type default))
  (layer "Edge.Cuts"))
 (segment (start 154.35 99.2749) (end 152.9749 100.65) (width 0.2) (layer "F.Cu") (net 3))
 (segment (start 154.35 98.18) (end 154.35 99.2749) (width 0.2) (layer "F.Cu") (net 3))
 (via blind (at 152.9749 100.65) (size 0.6) (drill 0.3) (layers "F.Cu" "B.Cu") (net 3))
 (segment (start 152.9749 107.4998) (end 150.4751 105) (width 0.2) (layer "B.Cu") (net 3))
 (segment (start 150.4751 105) (end 152.9749 102.5002) (width 0.2) (layer "B.Cu") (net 3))
 (segment (start 152.9749 109.35) (end 152.9749 107.4998) (width 0.2) (layer "B.Cu") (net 3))
 (segment (start 152.9749 102.5002) (end 152.9749 100.65) (width 0.2) (layer "B.Cu") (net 3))
 (via blind (at 155.18 111.5675) (size 0.6) (drill 0.3) (layers "F.Cu" "B.Cu") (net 8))
 (segment (start 155.3025 111.5675) (end 155.602031 111.267969) (width 0.2) (layer "B.Cu") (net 8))
 (segment (start 155.18 111.5675) (end 155.3025 111.5675) (width 0.2) (layer "B.Cu") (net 8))
 (segment (start 149.2249 110.2018) (end 150.5906 111.5675) (width 0.2) (layer "B.Cu") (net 8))
 (segment (start 149.2249 109.35) (end 149.2249 110.2018) (width 0.2) (layer "B.Cu") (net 8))
 (segment (start 150.5906 111.5675) (end 155.18 111.5675) (width 0.2) (layer "B.Cu") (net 8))
 (segment (start 155.602031 111.267969) (end 159.537969 111.267969) (width 0.2) (layer "B.Cu") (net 8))
 (segment (start 151.74 100.635) (end 151.725 100.65) (width 0.2) (layer "F.Cu") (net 1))
 (segment (start 155.18 113.3925) (end 151.725 109.9375) (width 0.2) (layer "F.Cu") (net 1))
 (segment (start 149.6825 98.12) (end 152.39 98.12) (width 0.2) (layer "F.Cu") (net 1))
 (segment (start 146.87 113.425) (end 147.65 113.425) (width 0.2) (layer "F.Cu") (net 1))
 (segment (start 142.537969 109.092969) (end 142.537969 107.767969) (width 0.2) (layer "F.Cu") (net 1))
 (segment (start 151.74 98.38) (end 151.74 100.635) (width 0.2) (layer "F.Cu") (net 1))
 (segment (start 152.39 98.12) (end 152.45 98.18) (width 0.2) (layer "F.Cu") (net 1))
 (segment (start 146.87 113.425) (end 142.537969 109.092969) (width 0.2) (layer "F.Cu") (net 1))
 (segment (start 151.94 98.18) (end 151.74 98.38) (width 0.2) (layer "F.Cu") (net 1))
 (segment (start 151.725 109.9375) (end 151.725 109.35) (width 0.2) (layer "F.Cu") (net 1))
 (segment (start 152.45 98.18) (end 151.94 98.18) (width 0.2) (layer "F.Cu") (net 1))
 (segment (start 147.65 113.425) (end 151.725 109.35) (width 0.2) (layer "F.Cu") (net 1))
 (via blind (at 151.725 109.35) (size 0.6) (drill 0.3) (layers "F.Cu" "B.Cu") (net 1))
 (via blind (at 151.725 100.65) (size 0.6) (drill 0.3) (layers "F.Cu" "B.Cu") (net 1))
 (segment (start 142.537969 107.767969) (end 144.7241 105.581838) (width 0.2) (layer "B.Cu") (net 1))
 (segment (start 144.7241 101.7989) (end 147.274 99.249) (width 0.2) (layer "B.Cu") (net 1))
 (segment (start 151.725 99.95) (end 151.725 100.65) (width 0.2) (layer "B.Cu") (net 1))
 (segment (start 144.7241 105.581838) (end 144.7241 101.7989) (width 0.2) (layer "B.Cu") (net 1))
 (segment (start 151.024 99.249) (end 151.725 99.95) (width 0.2) (layer "B.Cu") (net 1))
 (segment (start 147.274 99.249) (end 151.024 99.249) (width 0.2) (layer "B.Cu") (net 1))
 (via blind (at 146.87 111.6) (size 0.6) (drill 0.3) (layers "F.Cu" "B.Cu") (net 2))
 (segment (start 141.336969 107.270498) (end 144.3231 104.284367) (width 0.2) (layer "B.Cu") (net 2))
 (segment (start 153.2749 98.848) (end 158.336969 103.910069) (width 0.2) (layer "B.Cu") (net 2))
 (segment (start 141.336969 108.26544) (end 141.336969 107.270498) (width 0.2) (layer "B.Cu") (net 2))
 (segment (start 144.671529 111.6) (end 141.336969 108.26544) (width 0.2) (layer "B.Cu") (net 2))
 (segment (start 144.3231 101.6328) (end 147.1079 98.848) (width 0.2) (layer "B.Cu") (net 2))
 (segment (start 144.3231 104.284367) (end 144.3231 101.6328) (width 0.2) (layer "B.Cu") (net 2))
 (segment (start 147.975 109.35) (end 147.975 110.495) (width 0.2) (layer "B.Cu") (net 2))
 (segment (start 146.87 111.6) (end 144.671529 111.6) (width 0.2) (layer "B.Cu") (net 2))
 (segment (start 147.975 110.495) (end 146.87 111.6) (width 0.2) (layer "B.Cu") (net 2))
 (segment (start 158.336969 103.910069) (end 158.336969 106.566969) (width 0.2) (layer "B.Cu") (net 2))
 (segment (start 158.336969 106.566969) (end 159.537969 107.767969) (width 0.2) (layer "B.Cu") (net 2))
 (segment (start 147.1079 98.848) (end 153.2749 98.848) (width 0.2) (layer "B.Cu") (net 2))
 (via blind (at 147.8575 98.12) (size 0.6) (drill 0.3) (layers "F.Cu" "B.Cu") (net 5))
 (segment (start 145.185938 98.12) (end 147.8575 98.12) (width 0.2) (layer "B.Cu") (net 5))
 (segment (start 142.537969 100.767969) (end 145.185938 98.12) (width 0.2) (layer "B.Cu") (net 5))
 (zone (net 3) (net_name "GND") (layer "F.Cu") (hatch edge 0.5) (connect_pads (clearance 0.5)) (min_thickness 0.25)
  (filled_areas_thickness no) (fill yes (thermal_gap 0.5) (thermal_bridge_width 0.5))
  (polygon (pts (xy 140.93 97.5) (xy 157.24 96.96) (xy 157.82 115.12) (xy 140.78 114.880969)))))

